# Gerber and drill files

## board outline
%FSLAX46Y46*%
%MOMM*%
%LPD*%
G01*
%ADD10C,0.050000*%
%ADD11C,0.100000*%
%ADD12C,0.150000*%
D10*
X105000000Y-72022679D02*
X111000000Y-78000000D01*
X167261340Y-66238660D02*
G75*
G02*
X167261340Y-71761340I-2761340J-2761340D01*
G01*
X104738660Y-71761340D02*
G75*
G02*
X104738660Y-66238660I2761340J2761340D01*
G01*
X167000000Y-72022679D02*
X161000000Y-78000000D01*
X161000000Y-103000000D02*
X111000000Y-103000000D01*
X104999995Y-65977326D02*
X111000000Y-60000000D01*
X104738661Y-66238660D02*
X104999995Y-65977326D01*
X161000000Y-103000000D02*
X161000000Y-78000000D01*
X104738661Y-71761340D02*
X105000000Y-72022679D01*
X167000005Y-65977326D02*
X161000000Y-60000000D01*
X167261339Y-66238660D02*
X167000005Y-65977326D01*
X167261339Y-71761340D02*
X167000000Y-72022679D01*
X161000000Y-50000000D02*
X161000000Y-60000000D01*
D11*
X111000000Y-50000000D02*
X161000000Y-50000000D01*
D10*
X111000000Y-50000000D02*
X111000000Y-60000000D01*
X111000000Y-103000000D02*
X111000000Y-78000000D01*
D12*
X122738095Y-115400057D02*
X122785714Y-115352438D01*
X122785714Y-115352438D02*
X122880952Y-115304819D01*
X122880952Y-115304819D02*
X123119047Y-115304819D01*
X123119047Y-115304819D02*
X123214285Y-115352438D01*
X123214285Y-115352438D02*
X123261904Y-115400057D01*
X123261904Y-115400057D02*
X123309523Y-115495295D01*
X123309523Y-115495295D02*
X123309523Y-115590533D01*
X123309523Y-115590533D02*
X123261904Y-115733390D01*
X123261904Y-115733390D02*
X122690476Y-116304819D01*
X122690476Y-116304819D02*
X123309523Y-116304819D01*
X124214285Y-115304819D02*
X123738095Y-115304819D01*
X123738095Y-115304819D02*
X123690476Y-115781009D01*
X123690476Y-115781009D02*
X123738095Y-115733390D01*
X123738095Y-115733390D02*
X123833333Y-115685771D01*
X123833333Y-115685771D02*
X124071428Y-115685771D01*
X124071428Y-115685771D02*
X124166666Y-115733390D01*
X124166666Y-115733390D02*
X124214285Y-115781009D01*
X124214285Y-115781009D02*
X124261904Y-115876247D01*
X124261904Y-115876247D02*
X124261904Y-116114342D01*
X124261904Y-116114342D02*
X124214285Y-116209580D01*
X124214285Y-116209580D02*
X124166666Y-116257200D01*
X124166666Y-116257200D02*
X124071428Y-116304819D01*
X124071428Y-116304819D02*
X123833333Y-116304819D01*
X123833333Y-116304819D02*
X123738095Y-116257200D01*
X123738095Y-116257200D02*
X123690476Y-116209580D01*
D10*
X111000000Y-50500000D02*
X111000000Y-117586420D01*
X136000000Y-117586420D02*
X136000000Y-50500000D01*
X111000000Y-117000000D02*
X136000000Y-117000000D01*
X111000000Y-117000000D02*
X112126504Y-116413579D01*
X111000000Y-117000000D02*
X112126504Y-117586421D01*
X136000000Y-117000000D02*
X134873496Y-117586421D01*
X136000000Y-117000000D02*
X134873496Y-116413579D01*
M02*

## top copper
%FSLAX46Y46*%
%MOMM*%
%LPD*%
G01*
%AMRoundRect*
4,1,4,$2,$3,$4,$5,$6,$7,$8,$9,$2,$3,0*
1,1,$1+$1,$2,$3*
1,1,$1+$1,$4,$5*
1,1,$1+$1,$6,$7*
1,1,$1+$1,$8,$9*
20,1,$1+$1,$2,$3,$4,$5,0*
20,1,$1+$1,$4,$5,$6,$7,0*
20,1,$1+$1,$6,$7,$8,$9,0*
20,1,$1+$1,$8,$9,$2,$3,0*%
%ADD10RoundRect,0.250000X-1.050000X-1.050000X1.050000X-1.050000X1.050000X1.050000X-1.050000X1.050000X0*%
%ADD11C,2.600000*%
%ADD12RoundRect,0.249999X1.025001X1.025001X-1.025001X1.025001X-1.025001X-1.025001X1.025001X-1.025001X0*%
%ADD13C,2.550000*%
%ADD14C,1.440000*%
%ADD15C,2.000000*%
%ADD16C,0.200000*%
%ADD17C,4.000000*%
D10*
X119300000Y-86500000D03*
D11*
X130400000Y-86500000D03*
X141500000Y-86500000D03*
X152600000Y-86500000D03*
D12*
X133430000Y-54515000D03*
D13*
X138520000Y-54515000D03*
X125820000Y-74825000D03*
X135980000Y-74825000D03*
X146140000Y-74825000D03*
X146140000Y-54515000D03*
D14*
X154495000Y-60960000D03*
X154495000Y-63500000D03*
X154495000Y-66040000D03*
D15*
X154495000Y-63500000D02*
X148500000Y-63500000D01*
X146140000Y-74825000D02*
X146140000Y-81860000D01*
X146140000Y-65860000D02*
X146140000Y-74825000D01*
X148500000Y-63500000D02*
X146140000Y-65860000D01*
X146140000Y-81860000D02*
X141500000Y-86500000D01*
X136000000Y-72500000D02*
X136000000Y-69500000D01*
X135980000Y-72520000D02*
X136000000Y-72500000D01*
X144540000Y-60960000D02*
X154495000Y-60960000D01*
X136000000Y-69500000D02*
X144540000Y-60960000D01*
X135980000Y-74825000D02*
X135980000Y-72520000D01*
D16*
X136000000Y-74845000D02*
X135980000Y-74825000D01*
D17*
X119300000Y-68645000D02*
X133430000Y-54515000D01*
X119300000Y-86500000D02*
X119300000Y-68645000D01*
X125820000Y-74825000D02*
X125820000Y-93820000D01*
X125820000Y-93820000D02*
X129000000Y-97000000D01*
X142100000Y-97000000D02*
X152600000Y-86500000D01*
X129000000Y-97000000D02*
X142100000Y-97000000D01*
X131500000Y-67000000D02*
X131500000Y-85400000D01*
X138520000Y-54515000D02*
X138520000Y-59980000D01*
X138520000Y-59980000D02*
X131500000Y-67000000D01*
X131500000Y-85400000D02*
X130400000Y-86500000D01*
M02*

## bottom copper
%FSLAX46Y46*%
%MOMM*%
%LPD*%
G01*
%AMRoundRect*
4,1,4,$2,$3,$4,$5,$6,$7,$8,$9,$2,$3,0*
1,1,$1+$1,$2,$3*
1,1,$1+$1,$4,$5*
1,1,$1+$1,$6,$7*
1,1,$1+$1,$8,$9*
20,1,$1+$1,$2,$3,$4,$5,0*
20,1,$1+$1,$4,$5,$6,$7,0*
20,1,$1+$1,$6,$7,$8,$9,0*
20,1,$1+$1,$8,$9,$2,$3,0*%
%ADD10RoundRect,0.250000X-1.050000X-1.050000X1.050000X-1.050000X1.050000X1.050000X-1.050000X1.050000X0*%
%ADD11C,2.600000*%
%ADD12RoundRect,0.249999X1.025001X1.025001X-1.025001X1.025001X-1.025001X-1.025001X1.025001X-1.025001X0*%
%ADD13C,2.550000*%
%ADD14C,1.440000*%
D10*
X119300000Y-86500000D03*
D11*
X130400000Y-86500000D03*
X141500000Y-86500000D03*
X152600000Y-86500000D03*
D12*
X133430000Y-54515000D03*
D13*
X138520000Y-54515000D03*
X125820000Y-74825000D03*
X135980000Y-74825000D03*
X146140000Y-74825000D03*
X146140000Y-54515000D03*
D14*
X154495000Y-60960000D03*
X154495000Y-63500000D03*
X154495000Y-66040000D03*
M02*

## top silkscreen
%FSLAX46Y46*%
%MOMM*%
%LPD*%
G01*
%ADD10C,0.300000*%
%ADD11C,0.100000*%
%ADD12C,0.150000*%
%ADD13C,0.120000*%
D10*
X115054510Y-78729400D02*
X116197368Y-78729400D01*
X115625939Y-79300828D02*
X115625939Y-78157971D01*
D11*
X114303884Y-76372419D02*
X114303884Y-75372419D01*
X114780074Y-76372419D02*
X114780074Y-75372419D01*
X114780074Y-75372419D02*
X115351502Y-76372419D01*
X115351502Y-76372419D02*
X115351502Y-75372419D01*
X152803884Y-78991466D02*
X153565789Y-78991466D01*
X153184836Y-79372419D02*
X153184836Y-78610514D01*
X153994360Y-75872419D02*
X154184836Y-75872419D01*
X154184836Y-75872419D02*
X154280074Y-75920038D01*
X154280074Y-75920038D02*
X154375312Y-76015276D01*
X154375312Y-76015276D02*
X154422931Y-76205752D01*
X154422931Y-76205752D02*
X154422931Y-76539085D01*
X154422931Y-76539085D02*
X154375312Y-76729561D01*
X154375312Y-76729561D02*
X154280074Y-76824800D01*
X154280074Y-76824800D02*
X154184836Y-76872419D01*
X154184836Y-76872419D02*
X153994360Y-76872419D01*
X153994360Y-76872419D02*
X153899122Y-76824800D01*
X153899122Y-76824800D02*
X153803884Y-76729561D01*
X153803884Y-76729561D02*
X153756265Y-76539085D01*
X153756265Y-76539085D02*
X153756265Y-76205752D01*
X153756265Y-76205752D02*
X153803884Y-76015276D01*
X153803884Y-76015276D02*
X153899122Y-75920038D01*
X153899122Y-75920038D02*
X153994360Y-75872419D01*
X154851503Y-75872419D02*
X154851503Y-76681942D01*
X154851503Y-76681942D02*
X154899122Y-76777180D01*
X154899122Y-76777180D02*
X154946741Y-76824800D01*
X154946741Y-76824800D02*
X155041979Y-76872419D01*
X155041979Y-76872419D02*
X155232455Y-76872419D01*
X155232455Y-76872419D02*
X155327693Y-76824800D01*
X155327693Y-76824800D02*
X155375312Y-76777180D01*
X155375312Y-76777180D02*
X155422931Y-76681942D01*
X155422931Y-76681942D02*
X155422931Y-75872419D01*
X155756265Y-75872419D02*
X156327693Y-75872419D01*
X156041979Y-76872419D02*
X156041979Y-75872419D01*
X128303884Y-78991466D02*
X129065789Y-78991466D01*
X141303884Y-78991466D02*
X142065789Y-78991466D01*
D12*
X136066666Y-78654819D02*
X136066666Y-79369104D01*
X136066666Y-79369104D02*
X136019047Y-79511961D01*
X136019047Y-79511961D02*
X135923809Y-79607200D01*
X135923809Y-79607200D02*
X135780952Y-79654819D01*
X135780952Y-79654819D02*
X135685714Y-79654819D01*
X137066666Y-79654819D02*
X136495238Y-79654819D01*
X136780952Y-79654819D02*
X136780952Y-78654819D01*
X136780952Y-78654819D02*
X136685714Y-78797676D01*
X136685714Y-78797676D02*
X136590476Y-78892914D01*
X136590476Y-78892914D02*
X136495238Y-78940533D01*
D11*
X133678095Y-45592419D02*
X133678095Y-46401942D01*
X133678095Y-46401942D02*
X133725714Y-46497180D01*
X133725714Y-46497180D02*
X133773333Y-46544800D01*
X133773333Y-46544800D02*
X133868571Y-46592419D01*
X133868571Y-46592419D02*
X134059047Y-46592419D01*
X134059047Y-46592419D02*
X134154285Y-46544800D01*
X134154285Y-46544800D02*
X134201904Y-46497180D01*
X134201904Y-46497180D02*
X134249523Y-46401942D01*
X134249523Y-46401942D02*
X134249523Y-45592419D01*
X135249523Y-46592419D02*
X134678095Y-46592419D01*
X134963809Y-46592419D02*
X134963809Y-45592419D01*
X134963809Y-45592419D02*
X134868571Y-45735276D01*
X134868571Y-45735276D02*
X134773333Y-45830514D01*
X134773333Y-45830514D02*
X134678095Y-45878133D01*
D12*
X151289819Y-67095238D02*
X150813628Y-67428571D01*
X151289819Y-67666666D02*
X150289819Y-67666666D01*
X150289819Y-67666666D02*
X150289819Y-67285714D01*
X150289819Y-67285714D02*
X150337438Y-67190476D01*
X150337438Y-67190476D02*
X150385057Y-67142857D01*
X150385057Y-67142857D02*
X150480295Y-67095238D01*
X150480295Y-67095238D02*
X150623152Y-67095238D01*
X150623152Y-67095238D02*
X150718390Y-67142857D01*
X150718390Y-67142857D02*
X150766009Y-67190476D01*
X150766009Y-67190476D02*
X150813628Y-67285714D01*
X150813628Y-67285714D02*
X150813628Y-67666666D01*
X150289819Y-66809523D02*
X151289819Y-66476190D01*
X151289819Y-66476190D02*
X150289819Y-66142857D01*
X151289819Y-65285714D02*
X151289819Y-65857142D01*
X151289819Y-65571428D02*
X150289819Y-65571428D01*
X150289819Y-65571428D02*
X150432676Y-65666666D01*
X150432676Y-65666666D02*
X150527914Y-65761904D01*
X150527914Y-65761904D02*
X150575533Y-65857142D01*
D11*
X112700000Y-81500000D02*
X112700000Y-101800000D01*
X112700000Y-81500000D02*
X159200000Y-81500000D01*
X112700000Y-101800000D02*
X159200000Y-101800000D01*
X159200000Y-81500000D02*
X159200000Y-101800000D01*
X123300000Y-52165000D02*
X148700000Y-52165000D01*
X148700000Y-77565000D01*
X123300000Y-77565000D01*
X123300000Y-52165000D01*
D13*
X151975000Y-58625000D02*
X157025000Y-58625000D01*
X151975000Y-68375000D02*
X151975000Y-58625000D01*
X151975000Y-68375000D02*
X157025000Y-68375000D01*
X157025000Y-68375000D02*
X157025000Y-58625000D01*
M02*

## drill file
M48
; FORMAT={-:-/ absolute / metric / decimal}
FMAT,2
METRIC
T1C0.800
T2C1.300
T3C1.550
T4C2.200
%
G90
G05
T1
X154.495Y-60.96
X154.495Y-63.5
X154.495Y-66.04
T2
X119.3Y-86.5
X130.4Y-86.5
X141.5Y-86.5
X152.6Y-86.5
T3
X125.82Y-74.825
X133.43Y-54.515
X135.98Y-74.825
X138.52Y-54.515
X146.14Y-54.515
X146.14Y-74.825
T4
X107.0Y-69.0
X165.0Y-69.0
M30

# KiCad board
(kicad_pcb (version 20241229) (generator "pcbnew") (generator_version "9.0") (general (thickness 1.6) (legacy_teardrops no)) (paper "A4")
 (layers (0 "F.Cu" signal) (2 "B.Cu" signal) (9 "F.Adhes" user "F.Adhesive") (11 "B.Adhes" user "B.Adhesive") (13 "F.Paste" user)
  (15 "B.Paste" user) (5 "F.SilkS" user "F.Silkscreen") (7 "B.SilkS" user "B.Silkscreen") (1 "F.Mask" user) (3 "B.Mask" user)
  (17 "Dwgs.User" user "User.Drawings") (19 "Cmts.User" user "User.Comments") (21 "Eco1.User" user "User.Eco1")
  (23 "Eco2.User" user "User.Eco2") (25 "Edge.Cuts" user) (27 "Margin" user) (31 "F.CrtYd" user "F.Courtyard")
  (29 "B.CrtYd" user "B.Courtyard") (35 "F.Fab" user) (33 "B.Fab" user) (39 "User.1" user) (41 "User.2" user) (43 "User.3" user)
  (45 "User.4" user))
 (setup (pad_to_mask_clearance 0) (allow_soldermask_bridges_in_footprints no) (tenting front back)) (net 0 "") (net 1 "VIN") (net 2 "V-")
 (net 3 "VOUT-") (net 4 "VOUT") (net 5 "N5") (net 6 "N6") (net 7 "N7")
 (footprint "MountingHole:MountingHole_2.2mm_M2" (layer "F.Cu") (at 165 69)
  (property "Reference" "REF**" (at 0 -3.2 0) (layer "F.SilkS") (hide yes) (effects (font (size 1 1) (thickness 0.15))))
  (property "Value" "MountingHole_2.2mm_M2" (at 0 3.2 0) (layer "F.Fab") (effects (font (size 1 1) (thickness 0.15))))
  (pad "" np_thru_hole circle (at 0 0) (size 2.2 2.2) (drill 2.2) (layers "*.Cu" "*.Mask")))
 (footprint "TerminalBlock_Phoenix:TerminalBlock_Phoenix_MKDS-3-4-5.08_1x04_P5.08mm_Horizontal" (layer "F.Cu") (at 119.3 86.5)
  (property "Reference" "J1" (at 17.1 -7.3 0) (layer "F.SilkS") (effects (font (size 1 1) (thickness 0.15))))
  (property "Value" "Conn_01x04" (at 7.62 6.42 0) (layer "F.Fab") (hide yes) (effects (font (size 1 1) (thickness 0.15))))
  (fp_line (start -6.6 -5) (end -6.6 15.3) (stroke (width 0.1) (type default)) (layer "F.SilkS"))
  (fp_line (start -6.6 -5) (end 39.9 -5) (stroke (width 0.1) (type default)) (layer "F.SilkS"))
  (fp_line (start -6.6 15.3) (end 39.9 15.3) (stroke (width 0.1) (type default)) (layer "F.SilkS"))
  (fp_line (start 39.9 -5) (end 39.9 15.3) (stroke (width 0.1) (type default)) (layer "F.SilkS"))
  (pad "1" thru_hole roundrect (at 0 0) (size 2.6 2.6) (drill 1.3) (layers "*.Cu" "*.Mask") (remove_unused_layers no)
   (roundrect_rratio 0.096154) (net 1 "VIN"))
  (pad "2" thru_hole circle (at 11.1 0) (size 2.6 2.6) (drill 1.3) (layers "*.Cu" "*.Mask") (remove_unused_layers no) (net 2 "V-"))
  (pad "3" thru_hole circle (at 22.2 0) (size 2.6 2.6) (drill 1.3) (layers "*.Cu" "*.Mask") (remove_unused_layers no) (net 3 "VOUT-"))
  (pad "4" thru_hole circle (at 33.3 0) (size 2.6 2.6) (drill 1.3) (layers "*.Cu" "*.Mask") (remove_unused_layers no) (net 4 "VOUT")))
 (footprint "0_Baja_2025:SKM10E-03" (layer "F.Cu") (at 134.44 46.635)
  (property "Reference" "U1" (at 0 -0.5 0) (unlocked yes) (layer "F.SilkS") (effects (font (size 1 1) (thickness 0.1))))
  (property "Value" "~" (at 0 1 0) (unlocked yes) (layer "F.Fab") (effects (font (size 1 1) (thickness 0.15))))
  (fp_rect (start -11.14 30.93) (end 14.26 5.53) (stroke (width 0.1) (type default)) (fill no) (layer "F.SilkS"))
  (pad "1" thru_hole roundrect (at -1.01 7.88 180) (size 2.55 2.55) (drill 1.55) (layers "*.Cu" "*.Mask") (remove_unused_layers no)
   (roundrect_rratio 0.098039) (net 1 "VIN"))
  (pad "2" thru_hole circle (at 4.08 7.88 180) (size 2.55 2.55) (drill 1.55) (layers "*.Cu" "*.Mask") (remove_unused_layers no) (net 2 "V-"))
  (pad "3" thru_hole circle (at -8.62 28.19 180) (size 2.55 2.55) (drill 1.55) (layers "*.Cu" "*.Mask") (remove_unused_layers no)
   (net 4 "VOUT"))
  (pad "4" thru_hole circle (at 1.54 28.19 180) (size 2.55 2.55) (drill 1.55) (layers "*.Cu" "*.Mask") (remove_unused_layers no)
   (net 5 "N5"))
  (pad "5" thru_hole circle (at 11.7 28.19 180) (size 2.55 2.55) (drill 1.55) (layers "*.Cu" "*.Mask") (remove_unused_layers no)
   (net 3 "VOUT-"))
  (pad "6" thru_hole circle (at 11.7 7.88 180) (size 2.55 2.55) (drill 1.55) (layers "*.Cu" "*.Mask") (remove_unused_layers no) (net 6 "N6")))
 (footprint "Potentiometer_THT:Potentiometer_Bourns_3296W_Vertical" (layer "F.Cu") (at 154.495 60.96 90)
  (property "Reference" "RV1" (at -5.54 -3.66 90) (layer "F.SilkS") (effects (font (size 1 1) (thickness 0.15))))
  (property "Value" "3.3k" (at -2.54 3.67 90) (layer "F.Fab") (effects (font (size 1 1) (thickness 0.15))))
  (fp_line (start 2.335 -2.52) (end 2.335 2.53) (stroke (width 0.12) (type solid)) (layer "F.SilkS"))
  (fp_line (start -7.415 -2.52) (end 2.335 -2.52) (stroke (width 0.12) (type solid)) (layer "F.SilkS"))
  (fp_line (start -7.415 -2.52) (end -7.415 2.53) (stroke (width 0.12) (type solid)) (layer "F.SilkS"))
  (fp_line (start -7.415 2.53) (end 2.335 2.53) (stroke (width 0.12) (type solid)) (layer "F.SilkS"))
  (pad "1" thru_hole circle (at 0 0 90) (size 1.44 1.44) (drill 0.8) (layers "*.Cu" "*.Mask") (remove_unused_layers no) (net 5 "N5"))
  (pad "2" thru_hole circle (at -2.54 0 90) (size 1.44 1.44) (drill 0.8) (layers "*.Cu" "*.Mask") (remove_unused_layers no) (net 3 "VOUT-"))
  (pad "3" thru_hole circle (at -5.08 0 90) (size 1.44 1.44) (drill 0.8) (layers "*.Cu" "*.Mask") (remove_unused_layers no) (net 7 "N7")))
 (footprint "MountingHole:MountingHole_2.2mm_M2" (layer "F.Cu") (at 107 69)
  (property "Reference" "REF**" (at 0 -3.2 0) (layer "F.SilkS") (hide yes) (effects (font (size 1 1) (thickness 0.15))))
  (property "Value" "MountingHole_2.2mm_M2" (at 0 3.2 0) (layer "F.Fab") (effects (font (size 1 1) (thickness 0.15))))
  (pad "" np_thru_hole circle (at 0 0) (size 2.2 2.2) (drill 2.2) (layers "*.Cu" "*.Mask")))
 (gr_line (start 105 72.022679) (end 111 78) (stroke (width 0.05) (type default)) (locked yes) (layer "Edge.Cuts"))
 (gr_arc (start 167.26134 66.23866) (mid 168.405124 69) (end 167.26134 71.76134) (stroke (width 0.05) (type default)) (locked yes)
  (layer "Edge.Cuts"))
 (gr_arc (start 104.73866 71.76134) (mid 103.594876 69) (end 104.73866 66.23866) (stroke (width 0.05) (type default)) (locked yes)
  (layer "Edge.Cuts"))
 (gr_line (start 167 72.022679) (end 161 78) (stroke (width 0.05) (type default)) (locked yes) (layer "Edge.Cuts"))
 (gr_line (start 161 103) (end 111 103) (stroke (width 0.05) (type default)) (locked yes) (layer "Edge.Cuts"))
 (gr_line (start 104.999995 65.977326) (end 111 60) (stroke (width 0.05) (type default)) (locked yes) (layer "Edge.Cuts"))
 (gr_line (start 104.738661 66.23866) (end 104.999995 65.977326) (stroke (width 0.05) (type default)) (locked yes) (layer "Edge.Cuts"))
 (gr_line (start 161 103) (end 161 78) (stroke (width 0.05) (type default)) (locked yes) (layer "Edge.Cuts"))
 (gr_line (start 104.738661 71.76134) (end 105 72.022679) (stroke (width 0.05) (type default)) (locked yes) (layer "Edge.Cuts"))
 (gr_line (start 167.000005 65.977326) (end 161 60) (stroke (width 0.05) (type default)) (locked yes) (layer "Edge.Cuts"))
 (gr_line (start 167.261339 66.23866) (end 167.000005 65.977326) (stroke (width 0.05) (type default)) (locked yes) (layer "Edge.Cuts"))
 (gr_line (start 167.261339 71.76134) (end 167 72.022679) (stroke (width 0.05) (type default)) (locked yes) (layer "Edge.Cuts"))
 (gr_line (start 161 50) (end 161 60) (stroke (width 0.05) (type default)) (locked yes) (layer "Edge.Cuts"))
 (gr_line (start 111 50) (end 161 50) (stroke (width 0.1) (type solid)) (locked yes) (layer "Edge.Cuts"))
 (gr_line (start 111 50) (end 111 60) (stroke (width 0.05) (type default)) (locked yes) (layer "Edge.Cuts"))
 (gr_line (start 111 103) (end 111 78) (stroke (width 0.05) (type default)) (locked yes) (layer "Edge.Cuts"))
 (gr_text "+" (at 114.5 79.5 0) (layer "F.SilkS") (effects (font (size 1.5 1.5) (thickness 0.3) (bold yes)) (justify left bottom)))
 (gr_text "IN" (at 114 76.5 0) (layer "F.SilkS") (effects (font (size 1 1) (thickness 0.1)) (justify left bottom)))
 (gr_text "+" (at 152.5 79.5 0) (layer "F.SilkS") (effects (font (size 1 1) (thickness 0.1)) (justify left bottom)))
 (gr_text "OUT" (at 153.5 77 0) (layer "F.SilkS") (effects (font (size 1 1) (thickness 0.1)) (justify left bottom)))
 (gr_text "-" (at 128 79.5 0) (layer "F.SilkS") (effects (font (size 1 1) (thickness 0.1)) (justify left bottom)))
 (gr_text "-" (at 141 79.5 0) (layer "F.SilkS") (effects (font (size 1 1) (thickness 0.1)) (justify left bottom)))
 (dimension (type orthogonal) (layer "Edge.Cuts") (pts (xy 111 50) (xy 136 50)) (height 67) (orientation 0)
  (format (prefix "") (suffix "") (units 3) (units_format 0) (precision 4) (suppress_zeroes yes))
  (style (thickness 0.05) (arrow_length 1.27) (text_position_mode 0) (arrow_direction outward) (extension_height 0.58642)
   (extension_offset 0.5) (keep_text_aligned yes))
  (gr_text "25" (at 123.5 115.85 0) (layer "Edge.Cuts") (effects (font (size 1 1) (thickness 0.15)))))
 (segment (start 154.495 63.5) (end 148.5 63.5) (width 2) (layer "F.Cu") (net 3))
 (segment (start 146.14 74.825) (end 146.14 81.86) (width 2) (layer "F.Cu") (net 3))
 (segment (start 146.14 65.86) (end 146.14 74.825) (width 2) (layer "F.Cu") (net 3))
 (segment (start 148.5 63.5) (end 146.14 65.86) (width 2) (layer "F.Cu") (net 3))
 (segment (start 146.14 81.86) (end 141.5 86.5) (width 2) (layer "F.Cu") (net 3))
 (segment (start 136 72.5) (end 136 69.5) (width 2) (layer "F.Cu") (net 5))
 (segment (start 135.98 72.52) (end 136 72.5) (width 2) (layer "F.Cu") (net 5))
 (segment (start 144.54 60.96) (end 154.495 60.96) (width 2) (layer "F.Cu") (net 5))
 (segment (start 136 69.5) (end 144.54 60.96) (width 2) (layer "F.Cu") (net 5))
 (segment (start 135.98 74.825) (end 135.98 72.52) (width 2) (layer "F.Cu") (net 5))
 (segment (start 136 74.845) (end 135.98 74.825) (width 0.2) (layer "F.Cu") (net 5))
 (segment (start 119.3 68.645) (end 133.43 54.515) (width 4) (layer "F.Cu") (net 1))
 (segment (start 119.3 86.5) (end 119.3 68.645) (width 4) (layer "F.Cu") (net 1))
 (segment (start 125.82 74.825) (end 125.82 93.82) (width 4) (layer "F.Cu") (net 4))
 (segment (start 125.82 93.82) (end 129 97) (width 4) (layer "F.Cu") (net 4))
 (segment (start 142.1 97) (end 152.6 86.5) (width 4) (layer "F.Cu") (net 4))
 (segment (start 129 97) (end 142.1 97) (width 4) (layer "F.Cu") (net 4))
 (segment (start 131.5 67) (end 131.5 85.4) (width 4) (layer "F.Cu") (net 2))
 (segment (start 138.52 54.515) (end 138.52 59.98) (width 4) (layer "F.Cu") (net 2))
 (segment (start 138.52 59.98) (end 131.5 67) (width 4) (layer "F.Cu") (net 2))
 (segment (start 131.5 85.4) (end 130.4 86.5) (width 4) (layer "F.Cu") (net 2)))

